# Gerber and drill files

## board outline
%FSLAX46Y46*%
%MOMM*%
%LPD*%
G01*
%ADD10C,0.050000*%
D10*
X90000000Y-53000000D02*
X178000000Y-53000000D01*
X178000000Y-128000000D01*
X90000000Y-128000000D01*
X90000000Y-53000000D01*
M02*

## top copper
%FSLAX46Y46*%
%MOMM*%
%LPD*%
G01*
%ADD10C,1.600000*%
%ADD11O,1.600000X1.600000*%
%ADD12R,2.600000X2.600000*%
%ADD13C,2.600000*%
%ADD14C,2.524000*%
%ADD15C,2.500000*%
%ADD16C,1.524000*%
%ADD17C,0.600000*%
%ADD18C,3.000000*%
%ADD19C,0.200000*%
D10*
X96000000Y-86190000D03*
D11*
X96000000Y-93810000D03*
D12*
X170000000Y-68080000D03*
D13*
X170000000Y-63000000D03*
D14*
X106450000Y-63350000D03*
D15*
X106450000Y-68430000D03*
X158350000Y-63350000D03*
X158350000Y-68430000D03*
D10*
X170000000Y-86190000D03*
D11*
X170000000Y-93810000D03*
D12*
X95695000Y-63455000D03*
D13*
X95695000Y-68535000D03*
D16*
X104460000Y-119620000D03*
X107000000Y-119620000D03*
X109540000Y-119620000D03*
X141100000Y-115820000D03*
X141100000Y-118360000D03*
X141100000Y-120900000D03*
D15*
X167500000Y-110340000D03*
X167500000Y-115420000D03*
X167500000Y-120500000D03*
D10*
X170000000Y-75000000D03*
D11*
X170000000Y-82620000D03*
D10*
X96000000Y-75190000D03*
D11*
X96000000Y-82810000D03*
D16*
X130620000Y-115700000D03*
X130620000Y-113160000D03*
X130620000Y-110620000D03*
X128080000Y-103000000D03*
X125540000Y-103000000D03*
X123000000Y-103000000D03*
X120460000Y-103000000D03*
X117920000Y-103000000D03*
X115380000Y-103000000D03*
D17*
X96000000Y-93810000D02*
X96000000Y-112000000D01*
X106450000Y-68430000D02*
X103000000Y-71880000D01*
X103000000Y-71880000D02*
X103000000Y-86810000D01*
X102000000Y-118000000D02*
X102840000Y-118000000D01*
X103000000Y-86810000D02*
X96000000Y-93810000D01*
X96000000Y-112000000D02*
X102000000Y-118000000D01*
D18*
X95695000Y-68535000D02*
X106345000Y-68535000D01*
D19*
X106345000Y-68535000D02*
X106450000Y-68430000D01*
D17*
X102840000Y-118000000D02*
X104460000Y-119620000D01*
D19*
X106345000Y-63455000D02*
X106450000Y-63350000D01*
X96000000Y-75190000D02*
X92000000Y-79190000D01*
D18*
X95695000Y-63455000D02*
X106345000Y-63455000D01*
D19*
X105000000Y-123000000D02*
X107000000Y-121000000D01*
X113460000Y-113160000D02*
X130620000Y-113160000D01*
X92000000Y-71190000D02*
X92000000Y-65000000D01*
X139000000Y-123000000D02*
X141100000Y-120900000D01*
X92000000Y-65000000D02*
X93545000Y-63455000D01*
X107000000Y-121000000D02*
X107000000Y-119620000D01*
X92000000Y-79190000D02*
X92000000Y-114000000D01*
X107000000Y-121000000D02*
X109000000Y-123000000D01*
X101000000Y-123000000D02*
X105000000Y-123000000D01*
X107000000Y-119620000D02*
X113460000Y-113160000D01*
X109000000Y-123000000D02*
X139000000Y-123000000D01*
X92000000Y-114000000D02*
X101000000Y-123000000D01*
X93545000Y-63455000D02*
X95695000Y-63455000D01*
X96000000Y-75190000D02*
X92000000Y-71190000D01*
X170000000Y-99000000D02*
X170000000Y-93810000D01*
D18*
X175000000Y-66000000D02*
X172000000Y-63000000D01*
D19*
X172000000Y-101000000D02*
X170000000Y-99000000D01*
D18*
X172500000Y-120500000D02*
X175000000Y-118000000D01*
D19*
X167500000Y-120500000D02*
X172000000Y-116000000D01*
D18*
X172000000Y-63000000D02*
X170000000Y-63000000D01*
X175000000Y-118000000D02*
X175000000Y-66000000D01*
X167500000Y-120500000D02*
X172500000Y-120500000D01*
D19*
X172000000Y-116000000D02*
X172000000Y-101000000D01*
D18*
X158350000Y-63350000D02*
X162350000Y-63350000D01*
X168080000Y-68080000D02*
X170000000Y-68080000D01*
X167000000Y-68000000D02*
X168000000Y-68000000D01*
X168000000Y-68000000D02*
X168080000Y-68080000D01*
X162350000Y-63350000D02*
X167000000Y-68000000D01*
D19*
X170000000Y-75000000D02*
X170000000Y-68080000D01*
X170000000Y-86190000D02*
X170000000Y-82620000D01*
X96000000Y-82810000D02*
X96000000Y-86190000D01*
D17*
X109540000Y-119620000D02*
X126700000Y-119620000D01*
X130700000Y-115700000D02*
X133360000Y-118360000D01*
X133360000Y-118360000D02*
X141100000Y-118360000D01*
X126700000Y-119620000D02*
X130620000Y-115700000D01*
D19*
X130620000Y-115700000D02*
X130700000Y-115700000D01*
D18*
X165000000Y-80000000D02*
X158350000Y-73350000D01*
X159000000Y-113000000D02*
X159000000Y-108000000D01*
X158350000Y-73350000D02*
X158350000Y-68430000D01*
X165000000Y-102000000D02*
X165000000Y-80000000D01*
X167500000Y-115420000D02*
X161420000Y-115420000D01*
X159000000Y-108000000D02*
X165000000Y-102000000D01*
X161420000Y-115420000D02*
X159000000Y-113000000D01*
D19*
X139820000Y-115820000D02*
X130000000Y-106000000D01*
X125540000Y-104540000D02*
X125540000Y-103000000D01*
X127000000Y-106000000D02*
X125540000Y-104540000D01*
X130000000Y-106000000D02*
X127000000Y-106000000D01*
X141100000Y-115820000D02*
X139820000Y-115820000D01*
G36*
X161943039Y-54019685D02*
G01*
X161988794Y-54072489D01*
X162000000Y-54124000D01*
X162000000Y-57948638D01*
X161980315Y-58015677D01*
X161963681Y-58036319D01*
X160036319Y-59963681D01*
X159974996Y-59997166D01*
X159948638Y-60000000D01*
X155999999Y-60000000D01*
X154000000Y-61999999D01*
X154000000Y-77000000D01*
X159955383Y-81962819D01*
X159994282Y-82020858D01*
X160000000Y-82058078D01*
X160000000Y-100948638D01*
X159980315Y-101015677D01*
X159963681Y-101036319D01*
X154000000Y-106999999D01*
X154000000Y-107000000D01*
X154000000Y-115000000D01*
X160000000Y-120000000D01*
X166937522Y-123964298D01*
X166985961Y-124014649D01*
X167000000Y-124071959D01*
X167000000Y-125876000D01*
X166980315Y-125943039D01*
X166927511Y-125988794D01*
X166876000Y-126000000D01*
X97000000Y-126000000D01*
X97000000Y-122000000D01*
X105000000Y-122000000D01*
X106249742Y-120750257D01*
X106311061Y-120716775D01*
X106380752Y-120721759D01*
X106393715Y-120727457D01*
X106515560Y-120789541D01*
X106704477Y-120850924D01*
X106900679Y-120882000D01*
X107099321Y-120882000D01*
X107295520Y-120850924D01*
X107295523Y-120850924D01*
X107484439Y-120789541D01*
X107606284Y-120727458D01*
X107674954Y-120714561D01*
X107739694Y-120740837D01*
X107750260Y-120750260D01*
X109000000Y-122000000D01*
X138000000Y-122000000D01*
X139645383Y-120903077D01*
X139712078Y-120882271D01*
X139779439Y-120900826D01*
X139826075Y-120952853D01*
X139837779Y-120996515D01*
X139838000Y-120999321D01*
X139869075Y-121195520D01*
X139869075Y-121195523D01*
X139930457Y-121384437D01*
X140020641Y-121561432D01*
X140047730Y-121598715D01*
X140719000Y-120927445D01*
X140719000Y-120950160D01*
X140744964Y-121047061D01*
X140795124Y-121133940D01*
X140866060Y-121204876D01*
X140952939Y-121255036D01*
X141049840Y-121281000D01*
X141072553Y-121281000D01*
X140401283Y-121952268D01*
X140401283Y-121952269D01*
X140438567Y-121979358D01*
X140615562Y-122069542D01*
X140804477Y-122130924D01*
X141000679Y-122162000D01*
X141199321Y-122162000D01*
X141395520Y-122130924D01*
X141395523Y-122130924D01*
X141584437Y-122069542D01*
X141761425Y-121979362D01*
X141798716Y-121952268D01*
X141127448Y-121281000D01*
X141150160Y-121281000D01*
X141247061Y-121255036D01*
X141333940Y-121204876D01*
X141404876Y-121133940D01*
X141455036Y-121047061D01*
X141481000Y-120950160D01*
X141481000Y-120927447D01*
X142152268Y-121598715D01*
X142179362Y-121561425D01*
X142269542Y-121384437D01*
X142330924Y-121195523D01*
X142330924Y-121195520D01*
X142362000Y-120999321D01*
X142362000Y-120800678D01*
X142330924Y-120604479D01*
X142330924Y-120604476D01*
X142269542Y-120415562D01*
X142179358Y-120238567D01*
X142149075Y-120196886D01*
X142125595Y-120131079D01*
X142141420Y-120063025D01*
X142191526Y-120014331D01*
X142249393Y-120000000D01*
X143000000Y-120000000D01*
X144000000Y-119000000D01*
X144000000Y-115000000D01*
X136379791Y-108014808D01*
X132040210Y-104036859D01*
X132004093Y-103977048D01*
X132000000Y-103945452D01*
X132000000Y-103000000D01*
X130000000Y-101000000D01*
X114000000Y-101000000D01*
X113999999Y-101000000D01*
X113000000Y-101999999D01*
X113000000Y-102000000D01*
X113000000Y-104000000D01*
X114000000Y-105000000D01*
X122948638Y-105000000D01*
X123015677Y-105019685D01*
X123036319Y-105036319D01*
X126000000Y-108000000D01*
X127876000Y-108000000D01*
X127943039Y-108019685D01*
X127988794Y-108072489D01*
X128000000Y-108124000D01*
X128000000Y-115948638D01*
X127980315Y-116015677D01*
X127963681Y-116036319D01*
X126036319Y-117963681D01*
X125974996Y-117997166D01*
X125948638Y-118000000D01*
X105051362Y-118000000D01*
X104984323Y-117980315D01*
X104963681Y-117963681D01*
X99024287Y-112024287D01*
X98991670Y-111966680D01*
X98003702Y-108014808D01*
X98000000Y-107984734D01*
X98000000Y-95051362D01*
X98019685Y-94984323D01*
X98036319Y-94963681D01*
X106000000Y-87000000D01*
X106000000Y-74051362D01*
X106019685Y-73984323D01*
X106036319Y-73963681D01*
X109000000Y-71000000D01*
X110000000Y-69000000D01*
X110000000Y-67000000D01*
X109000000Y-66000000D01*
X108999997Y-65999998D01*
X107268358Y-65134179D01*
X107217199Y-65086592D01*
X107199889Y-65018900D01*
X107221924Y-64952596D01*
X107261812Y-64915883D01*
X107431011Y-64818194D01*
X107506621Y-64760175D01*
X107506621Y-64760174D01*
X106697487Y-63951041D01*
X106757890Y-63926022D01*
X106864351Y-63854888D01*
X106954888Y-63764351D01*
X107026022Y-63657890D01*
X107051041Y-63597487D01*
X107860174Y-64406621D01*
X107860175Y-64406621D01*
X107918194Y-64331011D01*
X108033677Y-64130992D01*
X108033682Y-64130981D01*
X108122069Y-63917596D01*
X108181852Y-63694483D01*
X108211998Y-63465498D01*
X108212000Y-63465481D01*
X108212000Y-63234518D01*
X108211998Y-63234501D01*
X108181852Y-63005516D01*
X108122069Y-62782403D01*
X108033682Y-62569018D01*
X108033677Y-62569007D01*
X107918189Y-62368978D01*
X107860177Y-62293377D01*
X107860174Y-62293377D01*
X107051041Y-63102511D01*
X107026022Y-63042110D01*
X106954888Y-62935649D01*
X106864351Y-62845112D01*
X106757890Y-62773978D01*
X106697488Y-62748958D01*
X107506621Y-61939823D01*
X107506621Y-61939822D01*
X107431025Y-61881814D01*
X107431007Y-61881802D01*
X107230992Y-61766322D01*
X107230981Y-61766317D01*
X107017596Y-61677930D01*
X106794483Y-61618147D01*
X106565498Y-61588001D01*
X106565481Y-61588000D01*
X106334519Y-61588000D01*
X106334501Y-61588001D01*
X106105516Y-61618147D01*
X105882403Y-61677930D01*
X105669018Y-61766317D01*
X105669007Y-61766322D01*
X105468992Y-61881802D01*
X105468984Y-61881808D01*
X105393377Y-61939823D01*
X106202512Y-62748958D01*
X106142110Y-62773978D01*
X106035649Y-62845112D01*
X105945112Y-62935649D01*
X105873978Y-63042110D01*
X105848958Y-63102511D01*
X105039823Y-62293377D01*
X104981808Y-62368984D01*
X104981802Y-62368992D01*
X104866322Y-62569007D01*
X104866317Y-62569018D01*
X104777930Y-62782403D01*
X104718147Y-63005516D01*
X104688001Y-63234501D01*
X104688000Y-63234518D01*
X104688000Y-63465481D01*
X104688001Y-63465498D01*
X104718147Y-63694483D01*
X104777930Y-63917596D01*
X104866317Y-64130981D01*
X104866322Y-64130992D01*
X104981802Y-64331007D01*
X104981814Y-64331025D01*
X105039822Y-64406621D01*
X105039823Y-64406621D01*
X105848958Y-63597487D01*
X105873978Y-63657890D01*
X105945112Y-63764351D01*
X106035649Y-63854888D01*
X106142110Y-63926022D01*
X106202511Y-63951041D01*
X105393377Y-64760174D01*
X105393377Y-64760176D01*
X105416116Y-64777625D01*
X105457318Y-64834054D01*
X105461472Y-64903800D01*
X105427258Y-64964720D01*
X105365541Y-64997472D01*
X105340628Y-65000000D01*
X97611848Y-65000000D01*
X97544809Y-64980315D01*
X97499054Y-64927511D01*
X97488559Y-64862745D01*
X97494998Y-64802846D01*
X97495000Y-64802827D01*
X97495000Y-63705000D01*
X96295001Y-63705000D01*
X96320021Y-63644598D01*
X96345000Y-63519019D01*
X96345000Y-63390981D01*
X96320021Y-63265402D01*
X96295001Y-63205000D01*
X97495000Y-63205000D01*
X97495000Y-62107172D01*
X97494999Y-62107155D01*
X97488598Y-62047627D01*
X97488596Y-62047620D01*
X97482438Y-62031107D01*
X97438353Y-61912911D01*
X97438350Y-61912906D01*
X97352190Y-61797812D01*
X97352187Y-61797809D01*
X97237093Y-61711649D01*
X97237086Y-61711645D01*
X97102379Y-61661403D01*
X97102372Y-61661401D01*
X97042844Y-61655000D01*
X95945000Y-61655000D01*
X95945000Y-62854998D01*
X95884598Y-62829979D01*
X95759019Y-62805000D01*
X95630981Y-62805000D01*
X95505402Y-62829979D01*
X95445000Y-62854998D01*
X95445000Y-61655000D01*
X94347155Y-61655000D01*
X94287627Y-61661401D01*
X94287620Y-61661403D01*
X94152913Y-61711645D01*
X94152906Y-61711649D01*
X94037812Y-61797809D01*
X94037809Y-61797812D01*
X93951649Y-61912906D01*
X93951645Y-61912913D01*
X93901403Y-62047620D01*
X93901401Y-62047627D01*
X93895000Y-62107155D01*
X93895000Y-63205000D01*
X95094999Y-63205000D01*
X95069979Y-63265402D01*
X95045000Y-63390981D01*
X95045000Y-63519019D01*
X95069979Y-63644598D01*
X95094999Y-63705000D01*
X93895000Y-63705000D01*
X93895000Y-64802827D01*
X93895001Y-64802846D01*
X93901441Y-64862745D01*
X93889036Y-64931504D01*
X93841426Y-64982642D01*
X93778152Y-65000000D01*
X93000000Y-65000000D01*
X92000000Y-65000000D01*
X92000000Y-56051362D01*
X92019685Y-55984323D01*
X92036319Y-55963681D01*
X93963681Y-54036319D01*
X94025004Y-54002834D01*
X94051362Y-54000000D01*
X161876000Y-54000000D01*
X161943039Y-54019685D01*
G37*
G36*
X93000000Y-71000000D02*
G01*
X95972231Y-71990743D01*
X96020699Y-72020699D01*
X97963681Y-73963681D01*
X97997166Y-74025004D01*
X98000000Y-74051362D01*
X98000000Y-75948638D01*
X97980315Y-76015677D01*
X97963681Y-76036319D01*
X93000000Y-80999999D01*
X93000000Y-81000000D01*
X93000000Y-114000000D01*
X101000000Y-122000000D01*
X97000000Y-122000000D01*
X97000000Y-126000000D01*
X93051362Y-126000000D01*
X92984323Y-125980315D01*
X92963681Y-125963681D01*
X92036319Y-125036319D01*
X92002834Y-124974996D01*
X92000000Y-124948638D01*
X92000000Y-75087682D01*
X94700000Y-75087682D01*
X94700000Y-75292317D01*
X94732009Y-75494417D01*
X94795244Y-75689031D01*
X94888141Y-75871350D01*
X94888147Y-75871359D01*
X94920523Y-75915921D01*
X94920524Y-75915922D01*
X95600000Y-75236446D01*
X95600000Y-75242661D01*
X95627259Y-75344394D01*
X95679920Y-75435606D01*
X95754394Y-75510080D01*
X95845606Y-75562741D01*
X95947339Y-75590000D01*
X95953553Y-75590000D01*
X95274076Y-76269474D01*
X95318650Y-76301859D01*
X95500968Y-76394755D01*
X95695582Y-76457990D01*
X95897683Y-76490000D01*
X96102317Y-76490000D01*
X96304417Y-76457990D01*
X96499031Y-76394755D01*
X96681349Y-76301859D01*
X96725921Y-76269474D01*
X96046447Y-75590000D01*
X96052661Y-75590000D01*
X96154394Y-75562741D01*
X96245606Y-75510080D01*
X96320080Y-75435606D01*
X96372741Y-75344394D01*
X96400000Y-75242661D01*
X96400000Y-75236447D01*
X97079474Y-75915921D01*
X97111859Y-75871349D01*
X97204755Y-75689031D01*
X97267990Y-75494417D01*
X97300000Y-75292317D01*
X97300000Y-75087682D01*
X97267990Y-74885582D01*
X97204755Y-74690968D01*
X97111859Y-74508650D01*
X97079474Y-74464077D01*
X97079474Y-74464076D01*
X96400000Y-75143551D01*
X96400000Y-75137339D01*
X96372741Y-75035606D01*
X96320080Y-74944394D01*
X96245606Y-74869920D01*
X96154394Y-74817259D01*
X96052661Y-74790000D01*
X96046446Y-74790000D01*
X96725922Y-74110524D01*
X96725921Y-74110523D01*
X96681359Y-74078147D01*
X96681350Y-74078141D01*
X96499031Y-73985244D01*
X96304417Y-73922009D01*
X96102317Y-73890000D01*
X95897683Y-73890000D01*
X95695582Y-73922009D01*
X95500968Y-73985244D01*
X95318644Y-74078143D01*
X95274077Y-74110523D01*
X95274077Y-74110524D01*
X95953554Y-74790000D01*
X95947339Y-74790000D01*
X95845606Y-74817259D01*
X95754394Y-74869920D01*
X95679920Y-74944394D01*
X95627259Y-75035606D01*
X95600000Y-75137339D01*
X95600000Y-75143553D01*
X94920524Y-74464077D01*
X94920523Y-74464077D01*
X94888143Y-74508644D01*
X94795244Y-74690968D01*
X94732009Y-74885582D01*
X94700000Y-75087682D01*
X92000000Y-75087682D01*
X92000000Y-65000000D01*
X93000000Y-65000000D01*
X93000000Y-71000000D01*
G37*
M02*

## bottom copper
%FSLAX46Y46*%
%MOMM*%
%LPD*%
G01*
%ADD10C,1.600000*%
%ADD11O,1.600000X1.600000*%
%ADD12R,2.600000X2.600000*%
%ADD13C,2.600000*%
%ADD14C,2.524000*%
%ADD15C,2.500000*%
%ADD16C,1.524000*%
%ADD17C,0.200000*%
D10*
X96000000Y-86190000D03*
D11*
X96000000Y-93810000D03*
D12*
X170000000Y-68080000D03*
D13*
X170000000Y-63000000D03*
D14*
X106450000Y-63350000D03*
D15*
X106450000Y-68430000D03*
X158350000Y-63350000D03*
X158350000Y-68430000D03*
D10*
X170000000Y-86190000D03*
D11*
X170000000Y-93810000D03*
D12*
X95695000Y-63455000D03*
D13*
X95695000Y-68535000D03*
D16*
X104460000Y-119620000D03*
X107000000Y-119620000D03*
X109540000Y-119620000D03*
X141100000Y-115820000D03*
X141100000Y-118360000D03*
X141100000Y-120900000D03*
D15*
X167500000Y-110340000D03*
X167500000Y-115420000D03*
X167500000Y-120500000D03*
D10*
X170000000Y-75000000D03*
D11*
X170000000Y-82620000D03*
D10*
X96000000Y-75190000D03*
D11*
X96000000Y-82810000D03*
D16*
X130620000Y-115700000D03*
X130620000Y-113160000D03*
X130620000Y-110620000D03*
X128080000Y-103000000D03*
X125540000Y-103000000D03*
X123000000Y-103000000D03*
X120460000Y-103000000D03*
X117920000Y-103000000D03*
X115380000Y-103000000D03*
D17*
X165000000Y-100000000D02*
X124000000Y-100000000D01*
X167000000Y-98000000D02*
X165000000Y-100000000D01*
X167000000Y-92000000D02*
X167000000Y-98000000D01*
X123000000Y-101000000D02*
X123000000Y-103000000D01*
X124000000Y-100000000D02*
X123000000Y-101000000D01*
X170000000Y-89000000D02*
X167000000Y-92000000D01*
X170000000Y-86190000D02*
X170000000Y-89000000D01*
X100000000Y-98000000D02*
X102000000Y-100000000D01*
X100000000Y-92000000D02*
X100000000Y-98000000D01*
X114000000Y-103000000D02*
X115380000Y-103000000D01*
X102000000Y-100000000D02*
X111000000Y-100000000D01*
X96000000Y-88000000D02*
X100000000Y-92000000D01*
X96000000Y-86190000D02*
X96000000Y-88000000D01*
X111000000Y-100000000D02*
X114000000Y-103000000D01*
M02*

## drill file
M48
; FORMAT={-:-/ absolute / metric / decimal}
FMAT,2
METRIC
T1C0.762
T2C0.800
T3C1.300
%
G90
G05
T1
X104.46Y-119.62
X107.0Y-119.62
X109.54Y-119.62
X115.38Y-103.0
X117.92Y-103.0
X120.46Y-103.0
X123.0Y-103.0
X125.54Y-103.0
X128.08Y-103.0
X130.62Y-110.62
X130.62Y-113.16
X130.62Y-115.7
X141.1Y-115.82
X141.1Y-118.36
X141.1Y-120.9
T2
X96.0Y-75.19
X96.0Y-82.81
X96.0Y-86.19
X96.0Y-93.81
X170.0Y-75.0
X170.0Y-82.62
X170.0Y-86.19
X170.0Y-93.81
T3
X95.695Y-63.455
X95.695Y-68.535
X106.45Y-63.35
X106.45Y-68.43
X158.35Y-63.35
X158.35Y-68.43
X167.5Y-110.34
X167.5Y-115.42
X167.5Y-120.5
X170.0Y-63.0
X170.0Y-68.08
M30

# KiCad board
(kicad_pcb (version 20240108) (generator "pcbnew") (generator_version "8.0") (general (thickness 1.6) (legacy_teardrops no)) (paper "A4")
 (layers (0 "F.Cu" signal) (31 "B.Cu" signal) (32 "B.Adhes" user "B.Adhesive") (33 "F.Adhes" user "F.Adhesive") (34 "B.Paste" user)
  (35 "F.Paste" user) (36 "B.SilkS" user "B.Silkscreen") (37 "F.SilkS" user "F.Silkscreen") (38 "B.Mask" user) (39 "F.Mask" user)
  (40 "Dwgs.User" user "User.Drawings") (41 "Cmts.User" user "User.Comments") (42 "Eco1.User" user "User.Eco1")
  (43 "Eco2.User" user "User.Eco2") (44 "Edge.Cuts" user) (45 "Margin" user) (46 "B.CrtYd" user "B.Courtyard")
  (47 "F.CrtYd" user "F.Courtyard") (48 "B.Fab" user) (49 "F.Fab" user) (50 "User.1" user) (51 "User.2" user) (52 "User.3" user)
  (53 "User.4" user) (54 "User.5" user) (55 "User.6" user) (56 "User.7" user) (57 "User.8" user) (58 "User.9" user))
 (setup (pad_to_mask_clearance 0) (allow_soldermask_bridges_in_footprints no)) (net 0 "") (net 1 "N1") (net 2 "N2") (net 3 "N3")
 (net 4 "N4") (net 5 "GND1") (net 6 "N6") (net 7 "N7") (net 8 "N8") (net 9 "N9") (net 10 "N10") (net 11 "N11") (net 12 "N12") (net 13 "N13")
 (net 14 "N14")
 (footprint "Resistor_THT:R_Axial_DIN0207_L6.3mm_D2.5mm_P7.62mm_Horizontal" (layer "F.Cu") (at 96 86.19 -90)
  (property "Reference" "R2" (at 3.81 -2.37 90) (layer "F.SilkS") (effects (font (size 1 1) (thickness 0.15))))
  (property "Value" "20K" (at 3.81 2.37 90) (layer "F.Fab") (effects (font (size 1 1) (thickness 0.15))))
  (pad "1" thru_hole circle (at 0 0 270) (size 1.6 1.6) (drill 0.8) (layers "*.Cu" "*.Mask") (remove_unused_layers no) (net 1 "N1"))
  (pad "2" thru_hole oval (at 7.62 0 270) (size 1.6 1.6) (drill 0.8) (layers "*.Cu" "*.Mask") (remove_unused_layers no) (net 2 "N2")))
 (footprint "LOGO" (layer "F.Cu") (at 96 107)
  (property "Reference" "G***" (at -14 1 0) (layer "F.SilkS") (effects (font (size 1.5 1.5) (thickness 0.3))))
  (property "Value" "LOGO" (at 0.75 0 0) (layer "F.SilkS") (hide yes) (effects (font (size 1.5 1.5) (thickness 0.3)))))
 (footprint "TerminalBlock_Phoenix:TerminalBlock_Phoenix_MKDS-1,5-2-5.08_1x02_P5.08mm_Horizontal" (layer "F.Cu") (at 170 68.08 90)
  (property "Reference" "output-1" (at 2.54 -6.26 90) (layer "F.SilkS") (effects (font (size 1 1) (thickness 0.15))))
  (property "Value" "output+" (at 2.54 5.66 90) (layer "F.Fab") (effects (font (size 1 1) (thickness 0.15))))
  (pad "1" thru_hole rect (at 0 0 90) (size 2.6 2.6) (drill 1.3) (layers "*.Cu" "*.Mask") (remove_unused_layers no) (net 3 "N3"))
  (pad "2" thru_hole circle (at 5.08 0 90) (size 2.6 2.6) (drill 1.3) (layers "*.Cu" "*.Mask") (remove_unused_layers no) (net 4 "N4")))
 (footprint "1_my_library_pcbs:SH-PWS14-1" (layer "F.Cu") (at 131.55 76.05)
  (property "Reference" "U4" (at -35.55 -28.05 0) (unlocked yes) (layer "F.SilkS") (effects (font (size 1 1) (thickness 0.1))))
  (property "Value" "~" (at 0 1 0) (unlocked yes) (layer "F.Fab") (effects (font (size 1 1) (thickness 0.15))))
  (pad "1" thru_hole circle (at -25.1 -12.7) (size 2.524 2.524) (drill 1.3) (layers "*.Cu" "*.Mask") (remove_unused_layers no)
   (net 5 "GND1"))
  (pad "2" thru_hole circle (at -25.1 -7.62) (size 2.5 2.5) (drill 1.3) (layers "*.Cu" "*.Mask") (remove_unused_layers no) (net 2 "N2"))
  (pad "3" thru_hole circle (at 26.8 -12.7) (size 2.5 2.5) (drill 1.3) (layers "*.Cu" "*.Mask") (remove_unused_layers no) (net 3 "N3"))
  (pad "4" thru_hole circle (at 26.8 -7.62) (size 2.5 2.5) (drill 1.3) (layers "*.Cu" "*.Mask") (remove_unused_layers no) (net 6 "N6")))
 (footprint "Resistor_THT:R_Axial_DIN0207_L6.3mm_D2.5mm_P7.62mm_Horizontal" (layer "F.Cu") (at 170 86.19 -90)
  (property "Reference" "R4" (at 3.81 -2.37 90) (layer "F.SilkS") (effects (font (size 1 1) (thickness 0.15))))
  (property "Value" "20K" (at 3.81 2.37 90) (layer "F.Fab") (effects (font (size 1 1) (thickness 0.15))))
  (pad "1" thru_hole circle (at 0 0 270) (size 1.6 1.6) (drill 0.8) (layers "*.Cu" "*.Mask") (remove_unused_layers no) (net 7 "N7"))
  (pad "2" thru_hole oval (at 7.62 0 270) (size 1.6 1.6) (drill 0.8) (layers "*.Cu" "*.Mask") (remove_unused_layers no) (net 4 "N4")))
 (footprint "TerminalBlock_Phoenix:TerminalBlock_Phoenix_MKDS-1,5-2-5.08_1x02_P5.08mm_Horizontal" (layer "F.Cu") (at 95.695 63.455 -90)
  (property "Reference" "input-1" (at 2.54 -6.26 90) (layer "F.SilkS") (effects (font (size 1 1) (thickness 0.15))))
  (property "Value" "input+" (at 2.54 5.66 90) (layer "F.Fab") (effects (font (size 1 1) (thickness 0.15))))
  (pad "1" thru_hole rect (at 0 0 270) (size 2.6 2.6) (drill 1.3) (layers "*.Cu" "*.Mask") (remove_unused_layers no) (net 5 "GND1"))
  (pad "2" thru_hole circle (at 5.08 0 270) (size 2.6 2.6) (drill 1.3) (layers "*.Cu" "*.Mask") (remove_unused_layers no) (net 2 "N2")))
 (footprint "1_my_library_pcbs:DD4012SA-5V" (layer "F.Cu") (at 107 112 90)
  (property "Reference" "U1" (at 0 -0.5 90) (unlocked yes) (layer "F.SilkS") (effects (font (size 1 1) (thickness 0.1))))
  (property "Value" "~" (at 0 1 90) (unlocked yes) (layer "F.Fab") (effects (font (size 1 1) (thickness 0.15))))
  (pad "1" thru_hole circle (at -7.62 -2.54 90) (size 1.524 1.524) (drill 0.762) (layers "*.Cu" "*.Mask") (remove_unused_layers no)
   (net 2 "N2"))
  (pad "2" thru_hole circle (at -7.62 0 90) (size 1.524 1.524) (drill 0.762) (layers "*.Cu" "*.Mask") (remove_unused_layers no)
   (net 5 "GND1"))
  (pad "3" thru_hole circle (at -7.62 2.54 90) (size 1.524 1.524) (drill 0.762) (layers "*.Cu" "*.Mask") (remove_unused_layers no)
   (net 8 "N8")))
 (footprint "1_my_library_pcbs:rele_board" (layer "F.Cu") (at 152 115)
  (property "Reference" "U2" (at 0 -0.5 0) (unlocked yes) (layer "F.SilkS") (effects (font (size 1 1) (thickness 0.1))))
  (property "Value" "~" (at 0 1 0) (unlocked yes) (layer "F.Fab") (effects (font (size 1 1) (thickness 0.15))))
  (pad "1" thru_hole circle (at -10.9 0.82) (size 1.524 1.524) (drill 0.762) (layers "*.Cu" "*.Mask") (remove_unused_layers no) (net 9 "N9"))
  (pad "2" thru_hole circle (at -10.9 3.36) (size 1.524 1.524) (drill 0.762) (layers "*.Cu" "*.Mask") (remove_unused_layers no) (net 8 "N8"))
  (pad "3" thru_hole circle (at -10.9 5.9) (size 1.524 1.524) (drill 0.762) (layers "*.Cu" "*.Mask") (remove_unused_layers no)
   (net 5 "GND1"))
  (pad "4" thru_hole circle (at 15.5 -4.66) (size 2.5 2.5) (drill 1.3) (layers "*.Cu" "*.Mask") (remove_unused_layers no) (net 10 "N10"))
  (pad "5" thru_hole circle (at 15.5 0.42) (size 2.5 2.5) (drill 1.3) (layers "*.Cu" "*.Mask") (remove_unused_layers no) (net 6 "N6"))
  (pad "6" thru_hole circle (at 15.5 5.5) (size 2.5 2.5) (drill 1.3) (layers "*.Cu" "*.Mask") (remove_unused_layers no) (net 4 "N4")))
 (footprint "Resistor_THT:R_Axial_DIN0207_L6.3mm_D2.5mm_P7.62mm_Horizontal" (layer "F.Cu") (at 170 75 -90)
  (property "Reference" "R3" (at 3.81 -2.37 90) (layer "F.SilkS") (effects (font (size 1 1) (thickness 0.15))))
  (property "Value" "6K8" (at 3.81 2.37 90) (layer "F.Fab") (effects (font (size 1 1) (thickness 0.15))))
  (pad "1" thru_hole circle (at 0 0 270) (size 1.6 1.6) (drill 0.8) (layers "*.Cu" "*.Mask") (remove_unused_layers no) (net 3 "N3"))
  (pad "2" thru_hole oval (at 7.62 0 270) (size 1.6 1.6) (drill 0.8) (layers "*.Cu" "*.Mask") (remove_unused_layers no) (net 7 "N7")))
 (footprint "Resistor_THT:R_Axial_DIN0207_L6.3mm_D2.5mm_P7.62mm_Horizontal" (layer "F.Cu") (at 96 75.19 -90)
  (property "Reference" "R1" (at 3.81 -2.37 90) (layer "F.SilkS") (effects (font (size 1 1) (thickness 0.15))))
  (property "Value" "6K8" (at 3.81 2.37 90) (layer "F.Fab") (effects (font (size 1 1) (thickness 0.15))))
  (pad "1" thru_hole circle (at 0 0 270) (size 1.6 1.6) (drill 0.8) (layers "*.Cu" "*.Mask") (remove_unused_layers no) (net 5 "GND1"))
  (pad "2" thru_hole oval (at 7.62 0 270) (size 1.6 1.6) (drill 0.8) (layers "*.Cu" "*.Mask") (remove_unused_layers no) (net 1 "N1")))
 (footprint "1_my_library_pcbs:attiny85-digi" (layer "F.Cu") (at 123 113.16 90)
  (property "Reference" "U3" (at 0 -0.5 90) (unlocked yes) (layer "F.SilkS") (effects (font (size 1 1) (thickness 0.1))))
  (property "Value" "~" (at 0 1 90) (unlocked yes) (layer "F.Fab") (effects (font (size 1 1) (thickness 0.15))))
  (pad "1" thru_hole circle (at -2.54 7.62 90) (size 1.524 1.524) (drill 0.762) (layers "*.Cu" "*.Mask") (remove_unused_layers no)
   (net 8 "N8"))
  (pad "2" thru_hole circle (at 0 7.62 90) (size 1.524 1.524) (drill 0.762) (layers "*.Cu" "*.Mask") (remove_unused_layers no)
   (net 5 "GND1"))
  (pad "3" thru_hole circle (at 2.54 7.62 90) (size 1.524 1.524) (drill 0.762) (layers "*.Cu" "*.Mask") (remove_unused_layers no)
   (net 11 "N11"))
  (pad "4" thru_hole circle (at 10.16 5.08 90) (size 1.524 1.524) (drill 0.762) (layers "*.Cu" "*.Mask") (remove_unused_layers no)
   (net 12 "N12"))
  (pad "5" thru_hole circle (at 10.16 2.54 90) (size 1.524 1.524) (drill 0.762) (layers "*.Cu" "*.Mask") (remove_unused_layers no)
   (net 9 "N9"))
  (pad "6" thru_hole circle (at 10.16 0 90) (size 1.524 1.524) (drill 0.762) (layers "*.Cu" "*.Mask") (remove_unused_layers no) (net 7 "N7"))
  (pad "7" thru_hole circle (at 10.16 -2.54 90) (size 1.524 1.524) (drill 0.762) (layers "*.Cu" "*.Mask") (remove_unused_layers no)
   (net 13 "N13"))
  (pad "8" thru_hole circle (at 10.16 -5.08 90) (size 1.524 1.524) (drill 0.762) (layers "*.Cu" "*.Mask") (remove_unused_layers no)
   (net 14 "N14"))
  (pad "9" thru_hole circle (at 10.16 -7.62 90) (size 1.524 1.524) (drill 0.762) (layers "*.Cu" "*.Mask") (remove_unused_layers no)
   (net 1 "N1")))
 (gr_rect (start 90 53) (end 178 128) (stroke (width 0.05) (type default)) (fill none) (layer "Edge.Cuts"))
 (segment (start 96 93.81) (end 96 112) (width 0.6) (layer "F.Cu") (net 2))
 (segment (start 106.45 68.43) (end 103 71.88) (width 0.6) (layer "F.Cu") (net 2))
 (segment (start 103 71.88) (end 103 86.81) (width 0.6) (layer "F.Cu") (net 2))
 (segment (start 102 118) (end 102.84 118) (width 0.6) (layer "F.Cu") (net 2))
 (segment (start 103 86.81) (end 96 93.81) (width 0.6) (layer "F.Cu") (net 2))
 (segment (start 96 112) (end 102 118) (width 0.6) (layer "F.Cu") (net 2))
 (segment (start 95.695 68.535) (end 106.345 68.535) (width 3) (layer "F.Cu") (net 2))
 (segment (start 106.345 68.535) (end 106.45 68.43) (width 0.2) (layer "F.Cu") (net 2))
 (segment (start 102.84 118) (end 104.46 119.62) (width 0.6) (layer "F.Cu") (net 2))
 (segment (start 106.345 63.455) (end 106.45 63.35) (width 0.2) (layer "F.Cu") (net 5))
 (segment (start 96 75.19) (end 92 79.19) (width 0.2) (layer "F.Cu") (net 5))
 (segment (start 95.695 63.455) (end 106.345 63.455) (width 3) (layer "F.Cu") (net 5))
 (segment (start 105 123) (end 107 121) (width 0.2) (layer "F.Cu") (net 5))
 (segment (start 113.46 113.16) (end 130.62 113.16) (width 0.2) (layer "F.Cu") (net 5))
 (segment (start 92 71.19) (end 92 65) (width 0.2) (layer "F.Cu") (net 5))
 (segment (start 139 123) (end 141.1 120.9) (width 0.2) (layer "F.Cu") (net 5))
 (segment (start 92 65) (end 93.545 63.455) (width 0.2) (layer "F.Cu") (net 5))
 (segment (start 107 121) (end 107 119.62) (width 0.2) (layer "F.Cu") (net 5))
 (segment (start 92 79.19) (end 92 114) (width 0.2) (layer "F.Cu") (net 5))
 (segment (start 107 121) (end 109 123) (width 0.2) (layer "F.Cu") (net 5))
 (segment (start 101 123) (end 105 123) (width 0.2) (layer "F.Cu") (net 5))
 (segment (start 107 119.62) (end 113.46 113.16) (width 0.2) (layer "F.Cu") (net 5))
 (segment (start 109 123) (end 139 123) (width 0.2) (layer "F.Cu") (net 5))
 (segment (start 92 114) (end 101 123) (width 0.2) (layer "F.Cu") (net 5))
 (segment (start 93.545 63.455) (end 95.695 63.455) (width 0.2) (layer "F.Cu") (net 5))
 (segment (start 96 75.19) (end 92 71.19) (width 0.2) (layer "F.Cu") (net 5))
 (segment (start 170 99) (end 170 93.81) (width 0.2) (layer "F.Cu") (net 4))
 (segment (start 175 66) (end 172 63) (width 3) (layer "F.Cu") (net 4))
 (segment (start 172 101) (end 170 99) (width 0.2) (layer "F.Cu") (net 4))
 (segment (start 172.5 120.5) (end 175 118) (width 3) (layer "F.Cu") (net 4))
 (segment (start 167.5 120.5) (end 172 116) (width 0.2) (layer "F.Cu") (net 4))
 (segment (start 172 63) (end 170 63) (width 3) (layer "F.Cu") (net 4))
 (segment (start 175 118) (end 175 66) (width 3) (layer "F.Cu") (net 4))
 (segment (start 167.5 120.5) (end 172.5 120.5) (width 3) (layer "F.Cu") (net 4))
 (segment (start 172 116) (end 172 101) (width 0.2) (layer "F.Cu") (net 4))
 (segment (start 158.35 63.35) (end 162.35 63.35) (width 3) (layer "F.Cu") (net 3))
 (segment (start 168.08 68.08) (end 170 68.08) (width 3) (layer "F.Cu") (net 3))
 (segment (start 167 68) (end 168 68) (width 3) (layer "F.Cu") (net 3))
 (segment (start 168 68) (end 168.08 68.08) (width 3) (layer "F.Cu") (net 3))
 (segment (start 162.35 63.35) (end 167 68) (width 3) (layer "F.Cu") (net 3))
 (segment (start 170 75) (end 170 68.08) (width 0.2) (layer "F.Cu") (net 3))
 (segment (start 170 86.19) (end 170 82.62) (width 0.2) (layer "F.Cu") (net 7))
 (segment (start 165 100) (end 124 100) (width 0.2) (layer "B.Cu") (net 7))
 (segment (start 167 98) (end 165 100) (width 0.2) (layer "B.Cu") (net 7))
 (segment (start 167 92) (end 167 98) (width 0.2) (layer "B.Cu") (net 7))
 (segment (start 123 101) (end 123 103) (width 0.2) (layer "B.Cu") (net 7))
 (segment (start 124 100) (end 123 101) (width 0.2) (layer "B.Cu") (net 7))
 (segment (start 170 89) (end 167 92) (width 0.2) (layer "B.Cu") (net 7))
 (segment (start 170 86.19) (end 170 89) (width 0.2) (layer "B.Cu") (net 7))
 (segment (start 96 82.81) (end 96 86.19) (width 0.2) (layer "F.Cu") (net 1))
 (segment (start 100 98) (end 102 100) (width 0.2) (layer "B.Cu") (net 1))
 (segment (start 100 92) (end 100 98) (width 0.2) (layer "B.Cu") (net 1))
 (segment (start 114 103) (end 115.38 103) (width 0.2) (layer "B.Cu") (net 1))
 (segment (start 102 100) (end 111 100) (width 0.2) (layer "B.Cu") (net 1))
 (segment (start 96 88) (end 100 92) (width 0.2) (layer "B.Cu") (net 1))
 (segment (start 96 86.19) (end 96 88) (width 0.2) (layer "B.Cu") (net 1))
 (segment (start 111 100) (end 114 103) (width 0.2) (layer "B.Cu") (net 1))
 (segment (start 109.54 119.62) (end 126.7 119.62) (width 0.6) (layer "F.Cu") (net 8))
 (segment (start 130.7 115.7) (end 133.36 118.36) (width 0.6) (layer "F.Cu") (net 8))
 (segment (start 133.36 118.36) (end 141.1 118.36) (width 0.6) (layer "F.Cu") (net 8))
 (segment (start 126.7 119.62) (end 130.62 115.7) (width 0.6) (layer "F.Cu") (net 8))
 (segment (start 130.62 115.7) (end 130.7 115.7) (width 0.2) (layer "F.Cu") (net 8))
 (segment (start 165 80) (end 158.35 73.35) (width 3) (layer "F.Cu") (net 6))
 (segment (start 159 113) (end 159 108) (width 3) (layer "F.Cu") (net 6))
 (segment (start 158.35 73.35) (end 158.35 68.43) (width 3) (layer "F.Cu") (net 6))
 (segment (start 165 102) (end 165 80) (width 3) (layer "F.Cu") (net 6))
 (segment (start 167.5 115.42) (end 161.42 115.42) (width 3) (layer "F.Cu") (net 6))
 (segment (start 159 108) (end 165 102) (width 3) (layer "F.Cu") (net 6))
 (segment (start 161.42 115.42) (end 159 113) (width 3) (layer "F.Cu") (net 6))
 (segment (start 139.82 115.82) (end 130 106) (width 0.2) (layer "F.Cu") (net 9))
 (segment (start 125.54 104.54) (end 125.54 103) (width 0.2) (layer "F.Cu") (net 9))
 (segment (start 127 106) (end 125.54 104.54) (width 0.2) (layer "F.Cu") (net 9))
 (segment (start 130 106) (end 127 106) (width 0.2) (layer "F.Cu") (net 9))
 (segment (start 141.1 115.82) (end 139.82 115.82) (width 0.2) (layer "F.Cu") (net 9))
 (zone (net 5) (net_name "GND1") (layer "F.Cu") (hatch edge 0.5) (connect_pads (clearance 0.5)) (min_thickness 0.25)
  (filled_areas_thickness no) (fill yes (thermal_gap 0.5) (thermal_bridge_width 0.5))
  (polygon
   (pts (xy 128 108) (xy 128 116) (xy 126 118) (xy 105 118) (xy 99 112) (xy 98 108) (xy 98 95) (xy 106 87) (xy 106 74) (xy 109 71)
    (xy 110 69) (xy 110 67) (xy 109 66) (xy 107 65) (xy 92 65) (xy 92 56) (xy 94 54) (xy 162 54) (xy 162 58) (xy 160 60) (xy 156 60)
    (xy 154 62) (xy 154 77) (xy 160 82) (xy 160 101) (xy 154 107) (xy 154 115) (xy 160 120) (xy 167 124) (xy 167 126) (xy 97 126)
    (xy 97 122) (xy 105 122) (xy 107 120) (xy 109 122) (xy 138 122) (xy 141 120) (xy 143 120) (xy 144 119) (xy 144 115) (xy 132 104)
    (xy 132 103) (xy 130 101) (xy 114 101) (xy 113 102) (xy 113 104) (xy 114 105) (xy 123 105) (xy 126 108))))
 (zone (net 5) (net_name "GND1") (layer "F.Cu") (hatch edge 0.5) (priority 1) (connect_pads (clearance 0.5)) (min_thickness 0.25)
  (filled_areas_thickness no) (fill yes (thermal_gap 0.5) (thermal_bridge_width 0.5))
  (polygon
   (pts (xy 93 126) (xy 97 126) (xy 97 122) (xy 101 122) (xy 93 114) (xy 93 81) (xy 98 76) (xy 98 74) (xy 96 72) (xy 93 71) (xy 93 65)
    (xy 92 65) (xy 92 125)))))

